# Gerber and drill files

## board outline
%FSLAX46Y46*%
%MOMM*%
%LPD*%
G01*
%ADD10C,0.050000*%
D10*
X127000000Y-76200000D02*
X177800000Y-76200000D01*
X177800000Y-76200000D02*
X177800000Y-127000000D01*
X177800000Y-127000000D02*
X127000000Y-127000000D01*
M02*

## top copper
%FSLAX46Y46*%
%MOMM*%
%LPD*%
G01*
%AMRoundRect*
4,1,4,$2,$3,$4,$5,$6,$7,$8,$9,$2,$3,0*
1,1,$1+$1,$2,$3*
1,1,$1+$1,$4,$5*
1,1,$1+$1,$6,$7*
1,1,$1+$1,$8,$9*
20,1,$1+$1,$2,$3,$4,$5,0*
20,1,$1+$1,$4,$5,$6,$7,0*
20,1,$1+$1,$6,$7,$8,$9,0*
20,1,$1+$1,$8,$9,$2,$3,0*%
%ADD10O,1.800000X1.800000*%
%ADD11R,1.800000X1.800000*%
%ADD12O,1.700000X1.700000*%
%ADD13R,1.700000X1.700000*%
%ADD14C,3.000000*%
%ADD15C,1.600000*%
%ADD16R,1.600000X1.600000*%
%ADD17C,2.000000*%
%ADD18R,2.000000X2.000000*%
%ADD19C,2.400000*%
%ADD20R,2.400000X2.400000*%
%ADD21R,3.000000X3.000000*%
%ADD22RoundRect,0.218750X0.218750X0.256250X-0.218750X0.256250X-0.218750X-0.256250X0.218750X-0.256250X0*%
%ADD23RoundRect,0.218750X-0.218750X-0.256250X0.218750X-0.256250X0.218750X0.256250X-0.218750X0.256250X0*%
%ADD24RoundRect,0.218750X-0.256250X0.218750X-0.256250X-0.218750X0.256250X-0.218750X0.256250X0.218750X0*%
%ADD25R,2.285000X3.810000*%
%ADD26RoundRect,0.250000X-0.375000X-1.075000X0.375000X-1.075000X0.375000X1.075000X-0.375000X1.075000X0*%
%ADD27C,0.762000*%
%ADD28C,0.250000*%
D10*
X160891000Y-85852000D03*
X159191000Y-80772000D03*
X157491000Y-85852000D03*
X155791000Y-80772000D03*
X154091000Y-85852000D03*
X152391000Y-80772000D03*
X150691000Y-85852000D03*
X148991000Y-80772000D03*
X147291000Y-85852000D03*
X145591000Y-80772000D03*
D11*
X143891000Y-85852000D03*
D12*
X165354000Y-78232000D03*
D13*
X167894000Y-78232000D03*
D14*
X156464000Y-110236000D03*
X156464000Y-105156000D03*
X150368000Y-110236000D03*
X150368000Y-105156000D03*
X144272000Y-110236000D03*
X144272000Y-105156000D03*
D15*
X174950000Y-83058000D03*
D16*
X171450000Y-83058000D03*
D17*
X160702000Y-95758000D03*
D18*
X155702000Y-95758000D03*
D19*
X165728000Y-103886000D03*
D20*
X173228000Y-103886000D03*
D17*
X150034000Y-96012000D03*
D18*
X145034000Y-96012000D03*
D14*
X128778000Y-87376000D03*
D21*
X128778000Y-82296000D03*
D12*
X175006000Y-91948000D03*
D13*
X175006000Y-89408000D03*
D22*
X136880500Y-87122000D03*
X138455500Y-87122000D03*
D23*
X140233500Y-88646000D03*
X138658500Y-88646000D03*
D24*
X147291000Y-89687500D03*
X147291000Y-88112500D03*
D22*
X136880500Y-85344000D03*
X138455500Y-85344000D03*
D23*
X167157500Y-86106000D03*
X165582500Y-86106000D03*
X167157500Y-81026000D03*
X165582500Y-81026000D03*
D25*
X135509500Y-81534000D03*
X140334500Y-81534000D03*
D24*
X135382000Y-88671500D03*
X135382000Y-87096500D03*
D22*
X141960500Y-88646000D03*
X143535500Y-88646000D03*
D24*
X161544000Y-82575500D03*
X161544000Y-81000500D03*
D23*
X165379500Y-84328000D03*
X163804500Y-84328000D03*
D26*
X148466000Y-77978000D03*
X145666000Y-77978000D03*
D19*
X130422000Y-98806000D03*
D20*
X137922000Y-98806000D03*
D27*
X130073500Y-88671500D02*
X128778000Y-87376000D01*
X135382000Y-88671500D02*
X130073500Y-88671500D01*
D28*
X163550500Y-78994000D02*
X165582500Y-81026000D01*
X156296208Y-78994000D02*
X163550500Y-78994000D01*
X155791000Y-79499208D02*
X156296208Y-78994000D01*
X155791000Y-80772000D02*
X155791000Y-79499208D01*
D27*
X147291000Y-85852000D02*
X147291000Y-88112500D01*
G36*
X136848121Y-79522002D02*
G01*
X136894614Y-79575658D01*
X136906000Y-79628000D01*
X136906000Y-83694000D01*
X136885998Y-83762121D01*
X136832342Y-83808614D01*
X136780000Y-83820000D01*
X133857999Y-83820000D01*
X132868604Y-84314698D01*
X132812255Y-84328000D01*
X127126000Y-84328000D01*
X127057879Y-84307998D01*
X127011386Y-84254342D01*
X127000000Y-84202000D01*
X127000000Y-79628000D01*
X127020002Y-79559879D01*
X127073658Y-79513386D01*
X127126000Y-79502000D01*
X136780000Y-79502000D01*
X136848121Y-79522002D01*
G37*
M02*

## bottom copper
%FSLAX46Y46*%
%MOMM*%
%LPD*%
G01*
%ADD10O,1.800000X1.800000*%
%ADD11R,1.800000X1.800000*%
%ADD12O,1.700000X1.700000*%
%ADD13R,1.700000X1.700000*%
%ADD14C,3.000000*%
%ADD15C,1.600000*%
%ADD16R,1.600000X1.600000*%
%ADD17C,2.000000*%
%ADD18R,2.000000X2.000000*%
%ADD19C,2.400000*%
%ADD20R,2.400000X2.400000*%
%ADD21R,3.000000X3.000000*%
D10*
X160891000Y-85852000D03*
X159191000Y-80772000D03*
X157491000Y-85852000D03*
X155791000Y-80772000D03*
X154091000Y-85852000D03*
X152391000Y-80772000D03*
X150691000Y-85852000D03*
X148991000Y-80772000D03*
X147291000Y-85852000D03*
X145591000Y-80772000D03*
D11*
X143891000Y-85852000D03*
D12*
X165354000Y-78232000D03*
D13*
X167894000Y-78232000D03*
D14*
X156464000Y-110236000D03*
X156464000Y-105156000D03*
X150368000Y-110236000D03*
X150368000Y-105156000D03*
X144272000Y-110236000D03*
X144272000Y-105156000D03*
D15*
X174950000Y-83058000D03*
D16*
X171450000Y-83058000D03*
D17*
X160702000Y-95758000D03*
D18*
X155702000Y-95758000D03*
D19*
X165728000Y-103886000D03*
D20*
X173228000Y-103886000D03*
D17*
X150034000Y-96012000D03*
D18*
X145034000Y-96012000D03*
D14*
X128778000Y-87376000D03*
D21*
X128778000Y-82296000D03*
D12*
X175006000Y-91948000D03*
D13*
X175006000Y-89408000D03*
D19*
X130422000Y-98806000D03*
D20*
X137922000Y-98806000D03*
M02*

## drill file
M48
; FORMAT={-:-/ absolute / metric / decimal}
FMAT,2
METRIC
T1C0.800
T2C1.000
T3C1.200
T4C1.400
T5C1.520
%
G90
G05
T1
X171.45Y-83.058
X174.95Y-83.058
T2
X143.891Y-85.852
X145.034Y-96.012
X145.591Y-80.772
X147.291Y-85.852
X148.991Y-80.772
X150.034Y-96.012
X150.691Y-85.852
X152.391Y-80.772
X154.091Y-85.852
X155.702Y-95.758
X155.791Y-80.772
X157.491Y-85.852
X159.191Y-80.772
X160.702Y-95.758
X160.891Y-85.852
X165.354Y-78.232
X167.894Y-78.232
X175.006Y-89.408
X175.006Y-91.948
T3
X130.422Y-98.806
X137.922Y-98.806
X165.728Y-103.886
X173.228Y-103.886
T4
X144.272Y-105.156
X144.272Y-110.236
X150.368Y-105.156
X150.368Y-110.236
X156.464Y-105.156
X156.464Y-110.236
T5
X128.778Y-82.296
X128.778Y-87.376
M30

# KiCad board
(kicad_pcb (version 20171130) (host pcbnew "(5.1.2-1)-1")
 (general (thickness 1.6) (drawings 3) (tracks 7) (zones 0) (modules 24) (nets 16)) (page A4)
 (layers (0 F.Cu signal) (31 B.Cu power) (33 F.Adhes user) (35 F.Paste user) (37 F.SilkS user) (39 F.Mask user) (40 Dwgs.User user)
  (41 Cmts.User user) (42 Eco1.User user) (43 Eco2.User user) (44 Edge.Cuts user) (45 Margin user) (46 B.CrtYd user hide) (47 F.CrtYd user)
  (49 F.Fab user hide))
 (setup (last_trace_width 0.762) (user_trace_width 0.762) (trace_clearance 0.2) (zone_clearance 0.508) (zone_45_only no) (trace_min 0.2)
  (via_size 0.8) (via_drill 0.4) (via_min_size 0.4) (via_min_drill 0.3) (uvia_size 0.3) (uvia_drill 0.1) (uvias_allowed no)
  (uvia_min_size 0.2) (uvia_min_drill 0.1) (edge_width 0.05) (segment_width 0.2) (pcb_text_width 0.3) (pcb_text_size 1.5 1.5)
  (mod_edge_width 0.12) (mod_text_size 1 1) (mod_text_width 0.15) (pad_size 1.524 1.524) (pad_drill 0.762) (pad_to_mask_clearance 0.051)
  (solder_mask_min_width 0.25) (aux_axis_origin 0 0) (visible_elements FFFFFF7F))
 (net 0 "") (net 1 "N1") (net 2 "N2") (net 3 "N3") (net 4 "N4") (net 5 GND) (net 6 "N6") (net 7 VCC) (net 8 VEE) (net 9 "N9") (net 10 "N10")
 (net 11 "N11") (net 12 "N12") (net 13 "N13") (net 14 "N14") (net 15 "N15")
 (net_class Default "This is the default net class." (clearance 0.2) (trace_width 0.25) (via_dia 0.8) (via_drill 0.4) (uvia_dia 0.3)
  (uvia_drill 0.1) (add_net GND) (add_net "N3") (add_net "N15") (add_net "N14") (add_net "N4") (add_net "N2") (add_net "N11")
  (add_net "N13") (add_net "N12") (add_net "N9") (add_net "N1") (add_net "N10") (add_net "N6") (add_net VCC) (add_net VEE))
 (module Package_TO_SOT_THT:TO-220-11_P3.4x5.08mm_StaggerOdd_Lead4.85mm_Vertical (layer F.Cu) (at 143.891 85.852)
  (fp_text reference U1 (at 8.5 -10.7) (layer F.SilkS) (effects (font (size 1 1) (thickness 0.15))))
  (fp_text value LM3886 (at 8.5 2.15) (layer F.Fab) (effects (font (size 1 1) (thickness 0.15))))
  (pad 11 thru_hole oval (at 17 0) (size 1.8 1.8) (drill 1) (layers *.Cu *.Mask) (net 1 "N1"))
  (pad 10 thru_hole oval (at 15.3 -5.08) (size 1.8 1.8) (drill 1) (layers *.Cu *.Mask) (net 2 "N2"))
  (pad 9 thru_hole oval (at 13.6 0) (size 1.8 1.8) (drill 1) (layers *.Cu *.Mask) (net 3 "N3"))
  (pad 8 thru_hole oval (at 11.9 -5.08) (size 1.8 1.8) (drill 1) (layers *.Cu *.Mask) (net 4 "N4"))
  (pad 7 thru_hole oval (at 10.2 0) (size 1.8 1.8) (drill 1) (layers *.Cu *.Mask) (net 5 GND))
  (pad 6 thru_hole oval (at 8.5 -5.08) (size 1.8 1.8) (drill 1) (layers *.Cu *.Mask) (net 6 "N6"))
  (pad 5 thru_hole oval (at 6.8 0) (size 1.8 1.8) (drill 1) (layers *.Cu *.Mask) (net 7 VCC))
  (pad 4 thru_hole oval (at 5.1 -5.08) (size 1.8 1.8) (drill 1) (layers *.Cu *.Mask) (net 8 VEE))
  (pad 3 thru_hole oval (at 3.4 0) (size 1.8 1.8) (drill 1) (layers *.Cu *.Mask) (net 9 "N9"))
  (pad 2 thru_hole oval (at 1.7 -5.08) (size 1.8 1.8) (drill 1) (layers *.Cu *.Mask) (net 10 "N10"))
  (pad 1 thru_hole rect (at 0 0) (size 1.8 1.8) (drill 1) (layers *.Cu *.Mask) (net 7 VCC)))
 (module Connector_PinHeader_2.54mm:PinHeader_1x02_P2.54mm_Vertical (layer F.Cu) (at 167.894 78.232 270)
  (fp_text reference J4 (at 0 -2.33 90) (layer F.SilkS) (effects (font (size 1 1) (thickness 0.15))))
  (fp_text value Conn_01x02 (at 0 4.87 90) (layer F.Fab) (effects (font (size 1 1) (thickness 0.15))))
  (pad 2 thru_hole oval (at 0 2.54 270) (size 1.7 1.7) (drill 1) (layers *.Cu *.Mask) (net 8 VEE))
  (pad 1 thru_hole rect (at 0 0 270) (size 1.7 1.7) (drill 1) (layers *.Cu *.Mask) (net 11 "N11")))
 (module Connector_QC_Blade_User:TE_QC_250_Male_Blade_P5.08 (layer F.Cu) (at 156.464 110.236 90)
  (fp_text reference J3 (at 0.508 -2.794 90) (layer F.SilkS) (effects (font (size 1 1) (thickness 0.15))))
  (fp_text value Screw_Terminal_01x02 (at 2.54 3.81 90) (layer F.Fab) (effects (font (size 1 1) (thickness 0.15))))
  (pad 1 thru_hole circle (at 0 0 90) (size 3 3) (drill 1.4) (layers *.Cu *.Mask) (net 8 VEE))
  (pad 2 thru_hole circle (at 5.08 0 90) (size 3 3) (drill 1.4) (layers *.Cu *.Mask) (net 8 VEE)))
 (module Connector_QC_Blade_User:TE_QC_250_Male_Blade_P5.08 (layer F.Cu) (at 150.368 110.236 90)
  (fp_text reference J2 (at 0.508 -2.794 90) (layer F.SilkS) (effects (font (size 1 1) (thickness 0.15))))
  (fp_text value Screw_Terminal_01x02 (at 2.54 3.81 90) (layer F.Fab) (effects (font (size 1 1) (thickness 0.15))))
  (pad 1 thru_hole circle (at 0 0 90) (size 3 3) (drill 1.4) (layers *.Cu *.Mask) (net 5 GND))
  (pad 2 thru_hole circle (at 5.08 0 90) (size 3 3) (drill 1.4) (layers *.Cu *.Mask) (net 5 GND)))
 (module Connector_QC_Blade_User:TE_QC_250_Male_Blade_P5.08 (layer F.Cu) (at 144.272 110.236 90)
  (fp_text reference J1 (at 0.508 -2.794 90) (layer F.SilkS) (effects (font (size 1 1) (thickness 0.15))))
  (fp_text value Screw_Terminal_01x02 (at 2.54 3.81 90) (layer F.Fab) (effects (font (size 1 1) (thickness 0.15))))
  (pad 1 thru_hole circle (at 0 0 90) (size 3 3) (drill 1.4) (layers *.Cu *.Mask) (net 7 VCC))
  (pad 2 thru_hole circle (at 5.08 0 90) (size 3 3) (drill 1.4) (layers *.Cu *.Mask) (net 7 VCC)))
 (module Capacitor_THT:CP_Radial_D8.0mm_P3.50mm (layer F.Cu) (at 171.45 83.058)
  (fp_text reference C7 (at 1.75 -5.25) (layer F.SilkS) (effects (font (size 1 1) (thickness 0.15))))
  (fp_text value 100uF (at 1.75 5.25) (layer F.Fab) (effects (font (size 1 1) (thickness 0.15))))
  (pad 2 thru_hole circle (at 3.5 0) (size 1.6 1.6) (drill 0.8) (layers *.Cu *.Mask) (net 5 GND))
  (pad 1 thru_hole rect (at 0 0) (size 1.6 1.6) (drill 0.8) (layers *.Cu *.Mask) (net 4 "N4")))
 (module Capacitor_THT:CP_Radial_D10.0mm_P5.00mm (layer F.Cu) (at 155.702 95.758)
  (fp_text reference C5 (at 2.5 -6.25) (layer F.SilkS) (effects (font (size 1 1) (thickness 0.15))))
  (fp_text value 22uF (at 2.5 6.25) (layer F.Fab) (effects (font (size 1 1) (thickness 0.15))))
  (pad 2 thru_hole circle (at 5 0) (size 2 2) (drill 1) (layers *.Cu *.Mask) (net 8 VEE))
  (pad 1 thru_hole rect (at 0 0) (size 2 2) (drill 1) (layers *.Cu *.Mask) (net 5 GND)))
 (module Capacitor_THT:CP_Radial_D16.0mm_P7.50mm (layer F.Cu) (at 173.228 103.886 180)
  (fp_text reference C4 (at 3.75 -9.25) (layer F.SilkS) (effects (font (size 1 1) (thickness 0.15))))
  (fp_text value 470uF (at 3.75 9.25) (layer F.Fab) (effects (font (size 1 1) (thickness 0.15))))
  (pad 2 thru_hole circle (at 7.5 0 180) (size 2.4 2.4) (drill 1.2) (layers *.Cu *.Mask) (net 8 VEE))
  (pad 1 thru_hole rect (at 0 0 180) (size 2.4 2.4) (drill 1.2) (layers *.Cu *.Mask) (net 5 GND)))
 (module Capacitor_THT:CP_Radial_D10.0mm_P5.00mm (layer F.Cu) (at 145.034 96.012)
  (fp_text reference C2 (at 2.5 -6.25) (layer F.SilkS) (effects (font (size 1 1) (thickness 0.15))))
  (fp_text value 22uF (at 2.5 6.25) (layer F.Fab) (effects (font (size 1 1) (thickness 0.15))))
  (pad 2 thru_hole circle (at 5 0) (size 2 2) (drill 1) (layers *.Cu *.Mask) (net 5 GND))
  (pad 1 thru_hole rect (at 0 0) (size 2 2) (drill 1) (layers *.Cu *.Mask) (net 7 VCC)))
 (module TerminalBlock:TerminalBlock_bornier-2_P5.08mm (layer F.Cu) (at 128.778 82.296 270)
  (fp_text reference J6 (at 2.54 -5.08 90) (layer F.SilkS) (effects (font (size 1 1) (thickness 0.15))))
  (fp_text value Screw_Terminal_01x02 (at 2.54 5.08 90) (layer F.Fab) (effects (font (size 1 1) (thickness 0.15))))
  (pad 2 thru_hole circle (at 5.08 0 270) (size 3 3) (drill 1.52) (layers *.Cu *.Mask) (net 5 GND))
  (pad 1 thru_hole rect (at 0 0 270) (size 3 3) (drill 1.52) (layers *.Cu *.Mask) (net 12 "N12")))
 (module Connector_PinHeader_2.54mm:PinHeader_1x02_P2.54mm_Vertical (layer F.Cu) (at 175.006 89.408)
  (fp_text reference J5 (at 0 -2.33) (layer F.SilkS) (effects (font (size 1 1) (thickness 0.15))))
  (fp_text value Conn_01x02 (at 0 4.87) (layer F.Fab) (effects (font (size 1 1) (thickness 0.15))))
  (pad 2 thru_hole oval (at 0 2.54) (size 1.7 1.7) (drill 1) (layers *.Cu *.Mask) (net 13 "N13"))
  (pad 1 thru_hole rect (at 0 0) (size 1.7 1.7) (drill 1) (layers *.Cu *.Mask) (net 5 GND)))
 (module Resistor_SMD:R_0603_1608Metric (layer F.Cu) (at 137.668 87.122 180)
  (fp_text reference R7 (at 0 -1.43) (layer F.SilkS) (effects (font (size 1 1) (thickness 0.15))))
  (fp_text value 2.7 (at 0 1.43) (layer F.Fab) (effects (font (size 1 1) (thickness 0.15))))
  (pad 2 smd roundrect (at 0.7875 0 180) (size 0.875 0.95) (layers F.Cu F.Paste F.Mask) (roundrect_rratio 0.25) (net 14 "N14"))
  (pad 1 smd roundrect (at -0.7875 0 180) (size 0.875 0.95) (layers F.Cu F.Paste F.Mask) (roundrect_rratio 0.25) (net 9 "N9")))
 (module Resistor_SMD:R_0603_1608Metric (layer F.Cu) (at 139.446 88.646)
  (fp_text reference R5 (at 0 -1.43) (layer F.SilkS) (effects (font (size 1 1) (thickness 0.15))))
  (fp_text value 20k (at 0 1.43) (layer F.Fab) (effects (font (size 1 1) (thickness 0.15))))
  (pad 2 smd roundrect (at 0.7875 0) (size 0.875 0.95) (layers F.Cu F.Paste F.Mask) (roundrect_rratio 0.25) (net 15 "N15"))
  (pad 1 smd roundrect (at -0.7875 0) (size 0.875 0.95) (layers F.Cu F.Paste F.Mask) (roundrect_rratio 0.25) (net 9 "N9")))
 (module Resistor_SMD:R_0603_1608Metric (layer F.Cu) (at 147.291 88.9 270)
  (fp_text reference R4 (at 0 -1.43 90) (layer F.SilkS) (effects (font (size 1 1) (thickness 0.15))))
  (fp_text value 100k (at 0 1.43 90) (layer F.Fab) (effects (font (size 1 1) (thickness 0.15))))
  (pad 2 smd roundrect (at 0.7875 0 270) (size 0.875 0.95) (layers F.Cu F.Paste F.Mask) (roundrect_rratio 0.25) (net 3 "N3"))
  (pad 1 smd roundrect (at -0.7875 0 270) (size 0.875 0.95) (layers F.Cu F.Paste F.Mask) (roundrect_rratio 0.25) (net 9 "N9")))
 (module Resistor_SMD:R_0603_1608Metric (layer F.Cu) (at 137.668 85.344 180)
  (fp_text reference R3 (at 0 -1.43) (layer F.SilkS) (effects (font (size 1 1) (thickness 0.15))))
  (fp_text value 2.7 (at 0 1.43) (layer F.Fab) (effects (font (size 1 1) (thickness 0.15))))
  (pad 2 smd roundrect (at 0.7875 0 180) (size 0.875 0.95) (layers F.Cu F.Paste F.Mask) (roundrect_rratio 0.25) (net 12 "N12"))
  (pad 1 smd roundrect (at -0.7875 0 180) (size 0.875 0.95) (layers F.Cu F.Paste F.Mask) (roundrect_rratio 0.25) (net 9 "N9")))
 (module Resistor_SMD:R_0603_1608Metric (layer F.Cu) (at 166.37 86.106)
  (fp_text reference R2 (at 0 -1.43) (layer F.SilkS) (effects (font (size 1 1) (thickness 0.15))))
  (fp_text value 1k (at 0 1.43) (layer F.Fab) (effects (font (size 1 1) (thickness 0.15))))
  (pad 2 smd roundrect (at 0.7875 0) (size 0.875 0.95) (layers F.Cu F.Paste F.Mask) (roundrect_rratio 0.25) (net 13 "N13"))
  (pad 1 smd roundrect (at -0.7875 0) (size 0.875 0.95) (layers F.Cu F.Paste F.Mask) (roundrect_rratio 0.25) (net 2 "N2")))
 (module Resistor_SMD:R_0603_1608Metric (layer F.Cu) (at 166.37 81.026)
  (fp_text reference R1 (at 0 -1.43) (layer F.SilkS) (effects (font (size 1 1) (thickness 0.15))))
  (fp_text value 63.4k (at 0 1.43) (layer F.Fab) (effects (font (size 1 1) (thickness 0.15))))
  (pad 2 smd roundrect (at 0.7875 0) (size 0.875 0.95) (layers F.Cu F.Paste F.Mask) (roundrect_rratio 0.25) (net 11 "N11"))
  (pad 1 smd roundrect (at -0.7875 0) (size 0.875 0.95) (layers F.Cu F.Paste F.Mask) (roundrect_rratio 0.25) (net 4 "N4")))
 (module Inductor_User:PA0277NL (layer F.Cu) (at 137.922 81.534 180)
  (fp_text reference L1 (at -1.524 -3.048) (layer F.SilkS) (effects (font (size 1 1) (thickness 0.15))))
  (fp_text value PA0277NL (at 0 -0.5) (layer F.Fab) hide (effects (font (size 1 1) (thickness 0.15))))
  (pad 2 smd rect (at 2.4125 0 180) (size 2.285 3.81) (layers F.Cu F.Paste F.Mask) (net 12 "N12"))
  (pad 1 smd rect (at -2.4125 0 180) (size 2.285 3.81) (layers F.Cu F.Paste F.Mask) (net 9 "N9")))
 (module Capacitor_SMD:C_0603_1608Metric (layer F.Cu) (at 135.382 87.884 270)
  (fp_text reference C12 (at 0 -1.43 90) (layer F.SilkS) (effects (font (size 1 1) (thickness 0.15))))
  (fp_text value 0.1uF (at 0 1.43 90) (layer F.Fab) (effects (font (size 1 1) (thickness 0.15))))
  (pad 2 smd roundrect (at 0.7875 0 270) (size 0.875 0.95) (layers F.Cu F.Paste F.Mask) (roundrect_rratio 0.25) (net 5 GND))
  (pad 1 smd roundrect (at -0.7875 0 270) (size 0.875 0.95) (layers F.Cu F.Paste F.Mask) (roundrect_rratio 0.25) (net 14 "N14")))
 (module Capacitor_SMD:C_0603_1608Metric (layer F.Cu) (at 142.748 88.646 180)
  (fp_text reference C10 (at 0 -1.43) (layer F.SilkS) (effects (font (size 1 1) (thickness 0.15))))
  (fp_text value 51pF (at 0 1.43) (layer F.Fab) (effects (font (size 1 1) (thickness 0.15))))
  (pad 2 smd roundrect (at 0.7875 0 180) (size 0.875 0.95) (layers F.Cu F.Paste F.Mask) (roundrect_rratio 0.25) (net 15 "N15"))
  (pad 1 smd roundrect (at -0.7875 0 180) (size 0.875 0.95) (layers F.Cu F.Paste F.Mask) (roundrect_rratio 0.25) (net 3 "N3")))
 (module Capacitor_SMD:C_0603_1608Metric (layer F.Cu) (at 161.544 81.788 270)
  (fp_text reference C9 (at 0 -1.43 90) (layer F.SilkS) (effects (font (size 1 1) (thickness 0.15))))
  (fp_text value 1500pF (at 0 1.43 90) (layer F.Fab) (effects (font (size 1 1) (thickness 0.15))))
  (pad 2 smd roundrect (at 0.7875 0 270) (size 0.875 0.95) (layers F.Cu F.Paste F.Mask) (roundrect_rratio 0.25) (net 5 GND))
  (pad 1 smd roundrect (at -0.7875 0 270) (size 0.875 0.95) (layers F.Cu F.Paste F.Mask) (roundrect_rratio 0.25) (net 2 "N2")))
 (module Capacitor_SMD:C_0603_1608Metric (layer F.Cu) (at 164.592 84.328)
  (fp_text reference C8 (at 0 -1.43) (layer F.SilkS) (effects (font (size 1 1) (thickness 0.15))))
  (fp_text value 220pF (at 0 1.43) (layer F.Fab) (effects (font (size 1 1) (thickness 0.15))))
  (pad 2 smd roundrect (at 0.7875 0) (size 0.875 0.95) (layers F.Cu F.Paste F.Mask) (roundrect_rratio 0.25) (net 2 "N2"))
  (pad 1 smd roundrect (at -0.7875 0) (size 0.875 0.95) (layers F.Cu F.Paste F.Mask) (roundrect_rratio 0.25) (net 3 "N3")))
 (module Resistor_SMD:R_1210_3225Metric (layer F.Cu) (at 147.066 77.978)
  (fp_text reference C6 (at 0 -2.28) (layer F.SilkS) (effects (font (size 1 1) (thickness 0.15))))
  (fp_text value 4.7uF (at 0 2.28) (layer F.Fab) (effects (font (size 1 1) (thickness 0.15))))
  (pad 2 smd roundrect (at 1.4 0) (size 1.25 2.65) (layers F.Cu F.Paste F.Mask) (roundrect_rratio 0.2) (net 8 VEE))
  (pad 1 smd roundrect (at -1.4 0) (size 1.25 2.65) (layers F.Cu F.Paste F.Mask) (roundrect_rratio 0.2) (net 5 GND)))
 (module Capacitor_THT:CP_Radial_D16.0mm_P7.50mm (layer F.Cu) (at 137.922 98.806 180)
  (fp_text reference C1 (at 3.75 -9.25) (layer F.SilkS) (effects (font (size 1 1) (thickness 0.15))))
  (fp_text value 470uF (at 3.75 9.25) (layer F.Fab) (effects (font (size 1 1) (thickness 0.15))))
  (pad 2 thru_hole circle (at 7.5 0 180) (size 2.4 2.4) (drill 1.2) (layers *.Cu *.Mask) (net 5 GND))
  (pad 1 thru_hole rect (at 0 0 180) (size 2.4 2.4) (drill 1.2) (layers *.Cu *.Mask) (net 7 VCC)))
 (gr_line (start 127 76.2) (end 177.8 76.2) (layer Edge.Cuts) (width 0.05))
 (gr_line (start 177.8 76.2) (end 177.8 127) (layer Edge.Cuts) (width 0.05))
 (gr_line (start 177.8 127) (end 127 127) (layer Edge.Cuts) (width 0.05))
 (segment (start 130.0735 88.6715) (end 128.778 87.376) (width 0.762) (layer F.Cu) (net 5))
 (segment (start 135.382 88.6715) (end 130.0735 88.6715) (width 0.762) (layer F.Cu) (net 5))
 (segment (start 163.5505 78.994) (end 165.5825 81.026) (width 0.25) (layer F.Cu) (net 4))
 (segment (start 156.296208 78.994) (end 163.5505 78.994) (width 0.25) (layer F.Cu) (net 4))
 (segment (start 155.791 79.499208) (end 156.296208 78.994) (width 0.25) (layer F.Cu) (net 4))
 (segment (start 155.791 80.772) (end 155.791 79.499208) (width 0.25) (layer F.Cu) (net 4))
 (segment (start 147.291 85.852) (end 147.291 88.1125) (width 0.762) (layer F.Cu) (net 9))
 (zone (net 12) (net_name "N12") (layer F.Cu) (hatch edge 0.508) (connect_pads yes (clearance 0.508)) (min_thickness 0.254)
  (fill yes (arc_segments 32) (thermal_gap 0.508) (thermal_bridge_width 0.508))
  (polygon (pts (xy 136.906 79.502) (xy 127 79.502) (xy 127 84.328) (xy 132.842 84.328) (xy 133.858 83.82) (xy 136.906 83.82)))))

